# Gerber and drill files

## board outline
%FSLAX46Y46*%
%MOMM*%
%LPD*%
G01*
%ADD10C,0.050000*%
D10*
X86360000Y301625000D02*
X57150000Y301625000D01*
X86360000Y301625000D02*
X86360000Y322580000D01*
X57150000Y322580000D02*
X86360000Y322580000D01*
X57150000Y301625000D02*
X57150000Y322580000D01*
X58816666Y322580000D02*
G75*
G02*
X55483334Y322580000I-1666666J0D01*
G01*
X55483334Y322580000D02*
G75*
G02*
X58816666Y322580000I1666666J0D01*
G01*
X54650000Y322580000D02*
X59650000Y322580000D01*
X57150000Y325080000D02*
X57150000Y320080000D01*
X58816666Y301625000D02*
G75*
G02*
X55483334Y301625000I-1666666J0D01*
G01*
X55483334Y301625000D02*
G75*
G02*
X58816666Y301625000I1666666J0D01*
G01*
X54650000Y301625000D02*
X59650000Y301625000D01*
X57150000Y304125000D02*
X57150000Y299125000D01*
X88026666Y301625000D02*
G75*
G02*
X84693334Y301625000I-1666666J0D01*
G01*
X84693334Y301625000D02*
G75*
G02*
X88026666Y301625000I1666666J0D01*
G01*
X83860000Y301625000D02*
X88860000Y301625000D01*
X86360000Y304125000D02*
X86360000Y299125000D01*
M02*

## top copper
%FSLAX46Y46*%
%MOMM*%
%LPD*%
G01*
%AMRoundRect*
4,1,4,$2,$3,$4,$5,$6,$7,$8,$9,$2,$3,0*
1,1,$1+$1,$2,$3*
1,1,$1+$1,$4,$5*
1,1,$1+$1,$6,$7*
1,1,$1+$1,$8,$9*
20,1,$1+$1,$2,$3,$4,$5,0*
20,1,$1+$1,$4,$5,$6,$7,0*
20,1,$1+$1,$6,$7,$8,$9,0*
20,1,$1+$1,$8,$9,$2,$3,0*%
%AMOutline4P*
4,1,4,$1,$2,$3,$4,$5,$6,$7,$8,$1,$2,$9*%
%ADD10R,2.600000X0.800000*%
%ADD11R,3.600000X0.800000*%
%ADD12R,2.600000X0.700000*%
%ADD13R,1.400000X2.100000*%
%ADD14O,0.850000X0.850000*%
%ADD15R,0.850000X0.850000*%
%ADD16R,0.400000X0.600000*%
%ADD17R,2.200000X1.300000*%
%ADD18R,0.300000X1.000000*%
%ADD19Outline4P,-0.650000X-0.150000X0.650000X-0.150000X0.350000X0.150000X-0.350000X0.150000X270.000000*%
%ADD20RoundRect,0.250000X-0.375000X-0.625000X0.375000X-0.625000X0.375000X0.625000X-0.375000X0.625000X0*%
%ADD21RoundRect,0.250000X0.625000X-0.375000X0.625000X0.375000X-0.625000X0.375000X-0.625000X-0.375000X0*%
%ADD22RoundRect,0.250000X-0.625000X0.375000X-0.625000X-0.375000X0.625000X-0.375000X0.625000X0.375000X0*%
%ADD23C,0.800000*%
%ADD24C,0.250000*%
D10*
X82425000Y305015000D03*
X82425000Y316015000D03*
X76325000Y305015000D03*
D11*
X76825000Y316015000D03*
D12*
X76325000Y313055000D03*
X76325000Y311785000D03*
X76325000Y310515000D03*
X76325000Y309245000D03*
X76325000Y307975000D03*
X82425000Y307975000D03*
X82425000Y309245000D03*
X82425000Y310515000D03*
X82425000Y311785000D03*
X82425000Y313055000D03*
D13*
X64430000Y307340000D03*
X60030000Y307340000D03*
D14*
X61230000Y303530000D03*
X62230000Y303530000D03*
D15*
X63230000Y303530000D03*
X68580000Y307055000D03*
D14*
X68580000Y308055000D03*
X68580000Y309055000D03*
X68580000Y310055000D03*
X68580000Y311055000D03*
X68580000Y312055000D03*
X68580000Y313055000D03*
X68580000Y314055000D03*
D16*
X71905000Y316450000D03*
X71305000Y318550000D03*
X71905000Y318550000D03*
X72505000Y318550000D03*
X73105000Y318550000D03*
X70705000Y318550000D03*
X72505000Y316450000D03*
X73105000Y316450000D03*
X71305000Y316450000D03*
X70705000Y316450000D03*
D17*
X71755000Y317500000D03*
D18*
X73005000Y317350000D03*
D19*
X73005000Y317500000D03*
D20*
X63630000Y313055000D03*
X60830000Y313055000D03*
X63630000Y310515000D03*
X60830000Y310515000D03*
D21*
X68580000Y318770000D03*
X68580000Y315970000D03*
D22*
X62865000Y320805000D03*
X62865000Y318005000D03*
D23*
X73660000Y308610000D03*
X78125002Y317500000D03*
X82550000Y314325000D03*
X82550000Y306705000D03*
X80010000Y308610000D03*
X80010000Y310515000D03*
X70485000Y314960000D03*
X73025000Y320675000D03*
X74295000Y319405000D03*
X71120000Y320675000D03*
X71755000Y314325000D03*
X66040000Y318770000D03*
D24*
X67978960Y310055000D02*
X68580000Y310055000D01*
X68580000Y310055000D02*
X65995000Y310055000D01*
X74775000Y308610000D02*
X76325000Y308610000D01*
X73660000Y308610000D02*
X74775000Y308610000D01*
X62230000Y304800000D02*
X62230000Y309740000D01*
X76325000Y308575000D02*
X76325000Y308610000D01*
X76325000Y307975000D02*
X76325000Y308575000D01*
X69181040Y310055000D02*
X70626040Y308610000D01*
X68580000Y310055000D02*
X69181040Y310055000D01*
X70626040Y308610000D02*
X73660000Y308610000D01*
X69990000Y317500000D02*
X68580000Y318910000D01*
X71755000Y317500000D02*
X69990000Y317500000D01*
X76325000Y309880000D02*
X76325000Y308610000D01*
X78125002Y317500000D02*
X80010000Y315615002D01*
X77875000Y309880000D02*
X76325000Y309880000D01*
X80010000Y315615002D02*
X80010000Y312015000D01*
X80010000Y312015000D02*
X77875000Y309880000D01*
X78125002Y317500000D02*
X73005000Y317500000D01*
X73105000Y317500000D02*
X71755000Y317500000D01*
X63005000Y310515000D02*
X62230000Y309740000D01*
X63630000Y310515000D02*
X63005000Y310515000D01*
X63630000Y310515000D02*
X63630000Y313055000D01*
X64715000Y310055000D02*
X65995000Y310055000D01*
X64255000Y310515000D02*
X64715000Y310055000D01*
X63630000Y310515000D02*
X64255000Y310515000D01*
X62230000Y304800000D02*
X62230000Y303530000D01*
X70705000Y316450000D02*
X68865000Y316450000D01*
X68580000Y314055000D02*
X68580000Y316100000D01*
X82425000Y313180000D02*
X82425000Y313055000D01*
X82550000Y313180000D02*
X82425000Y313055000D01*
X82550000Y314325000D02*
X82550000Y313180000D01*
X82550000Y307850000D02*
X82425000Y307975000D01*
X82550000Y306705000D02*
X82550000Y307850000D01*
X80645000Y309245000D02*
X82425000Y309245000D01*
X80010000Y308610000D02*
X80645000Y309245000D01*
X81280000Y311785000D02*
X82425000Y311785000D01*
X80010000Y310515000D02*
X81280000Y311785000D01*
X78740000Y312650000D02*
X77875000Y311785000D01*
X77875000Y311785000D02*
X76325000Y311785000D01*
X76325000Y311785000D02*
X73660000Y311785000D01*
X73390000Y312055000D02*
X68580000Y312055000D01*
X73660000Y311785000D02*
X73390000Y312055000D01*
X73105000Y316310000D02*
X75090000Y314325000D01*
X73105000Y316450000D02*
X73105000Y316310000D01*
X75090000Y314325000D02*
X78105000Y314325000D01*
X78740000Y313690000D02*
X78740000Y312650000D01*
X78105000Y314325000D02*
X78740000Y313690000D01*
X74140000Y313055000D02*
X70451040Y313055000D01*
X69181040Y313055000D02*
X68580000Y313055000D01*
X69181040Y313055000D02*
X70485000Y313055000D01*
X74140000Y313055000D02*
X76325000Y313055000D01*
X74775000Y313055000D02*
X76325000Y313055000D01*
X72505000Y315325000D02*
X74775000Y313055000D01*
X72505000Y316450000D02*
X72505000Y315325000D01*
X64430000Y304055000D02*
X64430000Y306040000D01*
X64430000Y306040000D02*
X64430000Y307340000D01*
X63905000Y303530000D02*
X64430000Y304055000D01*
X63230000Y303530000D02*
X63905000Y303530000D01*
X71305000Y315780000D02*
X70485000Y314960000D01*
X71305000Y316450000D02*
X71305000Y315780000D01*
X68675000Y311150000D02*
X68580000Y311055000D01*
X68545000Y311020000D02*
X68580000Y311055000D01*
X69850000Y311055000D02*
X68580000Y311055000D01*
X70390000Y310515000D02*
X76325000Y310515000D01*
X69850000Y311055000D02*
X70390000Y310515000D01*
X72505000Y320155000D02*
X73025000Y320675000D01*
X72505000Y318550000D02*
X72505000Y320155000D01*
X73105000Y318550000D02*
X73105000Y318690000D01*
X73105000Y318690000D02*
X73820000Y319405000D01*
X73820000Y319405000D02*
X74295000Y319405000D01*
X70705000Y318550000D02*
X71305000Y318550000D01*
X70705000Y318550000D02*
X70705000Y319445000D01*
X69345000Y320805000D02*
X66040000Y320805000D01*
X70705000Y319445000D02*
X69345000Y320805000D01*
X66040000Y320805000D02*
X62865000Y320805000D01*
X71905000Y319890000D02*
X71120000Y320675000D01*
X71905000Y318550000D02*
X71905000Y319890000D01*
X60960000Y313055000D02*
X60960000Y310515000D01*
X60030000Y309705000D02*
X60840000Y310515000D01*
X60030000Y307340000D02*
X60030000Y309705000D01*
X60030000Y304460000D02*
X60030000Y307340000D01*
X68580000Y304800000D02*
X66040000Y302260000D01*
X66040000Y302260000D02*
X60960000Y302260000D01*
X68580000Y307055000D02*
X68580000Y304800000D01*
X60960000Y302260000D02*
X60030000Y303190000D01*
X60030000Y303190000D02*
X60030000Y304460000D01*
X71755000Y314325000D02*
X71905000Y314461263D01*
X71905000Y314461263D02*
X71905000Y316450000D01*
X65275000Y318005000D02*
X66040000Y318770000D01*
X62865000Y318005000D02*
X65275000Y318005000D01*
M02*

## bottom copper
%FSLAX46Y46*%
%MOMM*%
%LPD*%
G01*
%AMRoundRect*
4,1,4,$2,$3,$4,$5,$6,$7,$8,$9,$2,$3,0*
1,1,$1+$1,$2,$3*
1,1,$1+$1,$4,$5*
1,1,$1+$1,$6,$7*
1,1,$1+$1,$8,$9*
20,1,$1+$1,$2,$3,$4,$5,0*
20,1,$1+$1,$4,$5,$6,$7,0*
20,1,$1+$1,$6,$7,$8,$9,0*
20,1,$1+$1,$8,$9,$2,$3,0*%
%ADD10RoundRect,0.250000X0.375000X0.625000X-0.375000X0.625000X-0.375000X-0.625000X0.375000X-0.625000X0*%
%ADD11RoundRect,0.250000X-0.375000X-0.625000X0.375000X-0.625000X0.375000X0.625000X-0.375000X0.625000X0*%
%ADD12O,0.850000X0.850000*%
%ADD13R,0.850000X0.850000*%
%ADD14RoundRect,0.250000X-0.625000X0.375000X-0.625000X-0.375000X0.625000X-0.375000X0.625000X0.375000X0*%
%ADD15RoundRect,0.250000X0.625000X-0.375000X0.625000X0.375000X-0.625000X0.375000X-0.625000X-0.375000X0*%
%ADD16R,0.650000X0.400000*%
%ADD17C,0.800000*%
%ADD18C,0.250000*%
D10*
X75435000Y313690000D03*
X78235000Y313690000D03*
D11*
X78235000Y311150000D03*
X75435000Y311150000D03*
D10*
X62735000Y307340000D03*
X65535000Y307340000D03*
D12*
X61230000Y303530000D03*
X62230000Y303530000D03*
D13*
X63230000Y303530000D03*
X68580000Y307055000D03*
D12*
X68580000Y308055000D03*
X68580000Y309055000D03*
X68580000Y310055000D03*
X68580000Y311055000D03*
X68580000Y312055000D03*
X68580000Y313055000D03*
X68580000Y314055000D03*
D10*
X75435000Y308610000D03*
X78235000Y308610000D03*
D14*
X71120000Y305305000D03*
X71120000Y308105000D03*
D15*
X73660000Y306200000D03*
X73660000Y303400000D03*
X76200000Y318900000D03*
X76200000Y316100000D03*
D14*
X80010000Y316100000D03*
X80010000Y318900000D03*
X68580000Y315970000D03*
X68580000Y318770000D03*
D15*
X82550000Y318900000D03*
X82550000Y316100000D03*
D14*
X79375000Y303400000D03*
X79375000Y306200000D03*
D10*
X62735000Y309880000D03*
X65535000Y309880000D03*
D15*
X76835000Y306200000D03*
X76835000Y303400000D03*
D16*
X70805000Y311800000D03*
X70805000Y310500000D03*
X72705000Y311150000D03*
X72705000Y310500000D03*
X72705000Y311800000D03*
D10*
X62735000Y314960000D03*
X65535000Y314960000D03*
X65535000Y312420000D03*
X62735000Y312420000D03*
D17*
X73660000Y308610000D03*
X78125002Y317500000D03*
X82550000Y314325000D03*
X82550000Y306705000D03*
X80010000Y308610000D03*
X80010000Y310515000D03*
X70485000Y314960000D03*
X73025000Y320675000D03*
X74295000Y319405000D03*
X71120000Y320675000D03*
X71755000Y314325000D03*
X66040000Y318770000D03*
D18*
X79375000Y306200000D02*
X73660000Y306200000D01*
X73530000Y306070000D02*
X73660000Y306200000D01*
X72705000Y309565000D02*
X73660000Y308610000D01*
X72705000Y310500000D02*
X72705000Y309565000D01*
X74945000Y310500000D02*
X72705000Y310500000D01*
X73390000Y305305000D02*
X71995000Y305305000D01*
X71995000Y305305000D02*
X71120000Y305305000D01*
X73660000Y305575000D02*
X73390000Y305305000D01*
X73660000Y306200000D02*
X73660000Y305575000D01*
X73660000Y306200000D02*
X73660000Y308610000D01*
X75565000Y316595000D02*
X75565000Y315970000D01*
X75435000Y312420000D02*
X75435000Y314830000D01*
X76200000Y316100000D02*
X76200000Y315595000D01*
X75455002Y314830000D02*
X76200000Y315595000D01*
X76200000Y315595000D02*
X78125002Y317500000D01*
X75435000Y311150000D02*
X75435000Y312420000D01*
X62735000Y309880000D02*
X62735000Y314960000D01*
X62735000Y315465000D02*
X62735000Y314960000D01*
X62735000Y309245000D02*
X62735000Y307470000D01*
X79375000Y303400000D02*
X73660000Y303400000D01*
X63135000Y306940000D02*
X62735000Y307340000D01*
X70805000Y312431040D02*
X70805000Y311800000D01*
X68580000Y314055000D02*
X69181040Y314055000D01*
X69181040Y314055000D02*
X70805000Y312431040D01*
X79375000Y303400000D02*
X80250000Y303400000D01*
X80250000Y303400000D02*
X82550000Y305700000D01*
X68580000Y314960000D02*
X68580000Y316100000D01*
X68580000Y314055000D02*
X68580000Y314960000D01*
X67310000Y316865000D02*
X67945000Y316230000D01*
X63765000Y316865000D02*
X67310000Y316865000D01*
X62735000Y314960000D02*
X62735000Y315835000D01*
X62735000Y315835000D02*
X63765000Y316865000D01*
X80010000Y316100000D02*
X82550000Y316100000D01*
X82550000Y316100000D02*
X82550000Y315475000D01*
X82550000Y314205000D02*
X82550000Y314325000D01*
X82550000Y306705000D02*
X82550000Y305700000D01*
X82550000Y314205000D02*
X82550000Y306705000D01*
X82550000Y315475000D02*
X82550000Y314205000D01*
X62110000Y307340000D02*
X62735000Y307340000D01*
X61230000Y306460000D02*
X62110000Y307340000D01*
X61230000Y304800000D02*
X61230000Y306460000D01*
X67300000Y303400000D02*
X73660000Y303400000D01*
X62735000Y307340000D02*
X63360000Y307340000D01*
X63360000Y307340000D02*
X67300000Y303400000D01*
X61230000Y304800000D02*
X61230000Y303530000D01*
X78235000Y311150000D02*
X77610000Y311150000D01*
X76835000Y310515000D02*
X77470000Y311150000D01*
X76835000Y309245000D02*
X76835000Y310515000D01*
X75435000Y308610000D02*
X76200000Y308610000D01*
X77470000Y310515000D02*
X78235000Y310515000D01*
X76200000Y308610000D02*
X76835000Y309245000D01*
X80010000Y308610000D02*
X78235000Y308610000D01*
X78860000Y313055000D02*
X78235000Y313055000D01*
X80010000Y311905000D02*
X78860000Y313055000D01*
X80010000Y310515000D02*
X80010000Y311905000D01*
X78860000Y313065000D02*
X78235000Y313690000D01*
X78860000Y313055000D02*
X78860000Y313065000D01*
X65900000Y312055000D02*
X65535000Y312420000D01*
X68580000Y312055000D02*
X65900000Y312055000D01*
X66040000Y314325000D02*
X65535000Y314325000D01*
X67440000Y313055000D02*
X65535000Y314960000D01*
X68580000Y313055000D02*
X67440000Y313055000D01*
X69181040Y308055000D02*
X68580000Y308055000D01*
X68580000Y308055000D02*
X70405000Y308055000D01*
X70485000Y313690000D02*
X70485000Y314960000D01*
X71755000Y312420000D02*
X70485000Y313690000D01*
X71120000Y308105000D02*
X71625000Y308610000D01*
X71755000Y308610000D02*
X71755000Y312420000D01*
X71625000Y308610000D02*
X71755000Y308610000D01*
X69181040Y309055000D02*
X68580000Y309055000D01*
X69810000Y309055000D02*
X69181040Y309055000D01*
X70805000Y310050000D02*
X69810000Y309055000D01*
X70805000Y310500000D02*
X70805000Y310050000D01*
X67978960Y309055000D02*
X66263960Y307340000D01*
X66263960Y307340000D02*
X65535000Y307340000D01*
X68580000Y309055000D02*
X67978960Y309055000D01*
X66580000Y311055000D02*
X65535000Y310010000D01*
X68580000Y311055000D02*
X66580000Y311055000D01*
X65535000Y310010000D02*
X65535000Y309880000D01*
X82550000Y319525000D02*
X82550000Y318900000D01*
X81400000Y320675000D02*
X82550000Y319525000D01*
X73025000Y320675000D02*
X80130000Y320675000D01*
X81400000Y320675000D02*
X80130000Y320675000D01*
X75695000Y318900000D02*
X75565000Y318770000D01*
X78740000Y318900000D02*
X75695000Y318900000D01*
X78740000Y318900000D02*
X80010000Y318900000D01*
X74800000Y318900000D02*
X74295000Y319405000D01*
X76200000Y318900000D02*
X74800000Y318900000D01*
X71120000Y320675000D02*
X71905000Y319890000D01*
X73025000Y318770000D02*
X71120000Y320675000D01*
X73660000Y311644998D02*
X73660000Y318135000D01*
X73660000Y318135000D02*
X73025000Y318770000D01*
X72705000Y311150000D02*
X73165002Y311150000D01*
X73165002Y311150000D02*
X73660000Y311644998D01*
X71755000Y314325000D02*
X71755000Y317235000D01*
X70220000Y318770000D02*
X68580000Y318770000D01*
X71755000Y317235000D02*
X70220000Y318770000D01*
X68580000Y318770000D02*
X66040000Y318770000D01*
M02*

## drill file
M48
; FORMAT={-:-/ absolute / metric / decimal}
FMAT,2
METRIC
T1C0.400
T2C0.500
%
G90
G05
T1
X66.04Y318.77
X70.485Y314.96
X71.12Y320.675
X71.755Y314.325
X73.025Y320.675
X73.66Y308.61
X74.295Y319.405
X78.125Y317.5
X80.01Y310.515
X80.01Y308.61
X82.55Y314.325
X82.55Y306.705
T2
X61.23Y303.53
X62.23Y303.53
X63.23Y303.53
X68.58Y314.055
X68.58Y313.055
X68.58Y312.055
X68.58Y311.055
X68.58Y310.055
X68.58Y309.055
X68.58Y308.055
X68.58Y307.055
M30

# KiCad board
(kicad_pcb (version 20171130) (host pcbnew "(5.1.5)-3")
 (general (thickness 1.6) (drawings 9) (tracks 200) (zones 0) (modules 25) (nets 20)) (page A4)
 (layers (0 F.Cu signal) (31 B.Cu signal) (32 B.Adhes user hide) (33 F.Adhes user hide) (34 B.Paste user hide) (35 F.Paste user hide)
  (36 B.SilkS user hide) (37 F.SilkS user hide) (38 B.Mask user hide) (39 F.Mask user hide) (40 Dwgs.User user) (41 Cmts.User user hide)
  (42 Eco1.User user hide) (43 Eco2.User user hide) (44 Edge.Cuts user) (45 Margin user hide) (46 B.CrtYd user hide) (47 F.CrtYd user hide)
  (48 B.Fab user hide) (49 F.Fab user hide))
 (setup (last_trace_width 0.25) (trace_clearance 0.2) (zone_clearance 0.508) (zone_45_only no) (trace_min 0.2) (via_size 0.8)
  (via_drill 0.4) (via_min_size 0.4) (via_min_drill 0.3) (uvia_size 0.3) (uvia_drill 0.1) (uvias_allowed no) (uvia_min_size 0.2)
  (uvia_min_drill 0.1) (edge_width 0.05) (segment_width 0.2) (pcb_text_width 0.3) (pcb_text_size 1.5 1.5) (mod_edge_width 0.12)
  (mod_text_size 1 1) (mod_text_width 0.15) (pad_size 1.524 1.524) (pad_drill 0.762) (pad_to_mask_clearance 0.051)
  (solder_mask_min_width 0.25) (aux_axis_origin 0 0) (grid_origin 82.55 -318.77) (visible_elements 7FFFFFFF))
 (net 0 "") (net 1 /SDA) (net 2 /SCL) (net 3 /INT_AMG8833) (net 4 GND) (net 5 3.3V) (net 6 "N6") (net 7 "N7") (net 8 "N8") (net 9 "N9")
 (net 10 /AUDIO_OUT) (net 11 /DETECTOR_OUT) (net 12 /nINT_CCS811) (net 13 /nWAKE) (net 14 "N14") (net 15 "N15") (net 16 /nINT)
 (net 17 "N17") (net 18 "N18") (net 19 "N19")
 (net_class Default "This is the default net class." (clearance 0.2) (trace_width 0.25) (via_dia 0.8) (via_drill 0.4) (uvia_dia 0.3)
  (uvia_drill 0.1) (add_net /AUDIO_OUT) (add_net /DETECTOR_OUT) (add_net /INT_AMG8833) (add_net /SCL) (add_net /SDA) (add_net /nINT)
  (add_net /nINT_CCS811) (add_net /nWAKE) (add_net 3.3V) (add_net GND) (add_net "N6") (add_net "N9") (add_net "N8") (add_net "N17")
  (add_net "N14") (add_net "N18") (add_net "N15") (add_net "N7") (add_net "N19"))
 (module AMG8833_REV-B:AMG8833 (layer F.Cu) (at 79.375 -310.515 270)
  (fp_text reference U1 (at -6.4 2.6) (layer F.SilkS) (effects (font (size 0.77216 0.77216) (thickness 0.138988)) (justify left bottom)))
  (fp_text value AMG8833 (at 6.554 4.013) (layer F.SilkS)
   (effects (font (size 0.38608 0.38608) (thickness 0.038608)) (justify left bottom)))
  (pad 8 smd rect (at 5.5 -3.05) (size 2.6 0.8) (layers F.Cu F.Paste F.Mask) (solder_mask_margin 0.0508))
  (pad 14 smd rect (at -5.5 -3.05) (size 2.6 0.8) (layers F.Cu F.Paste F.Mask) (solder_mask_margin 0.0508))
  (pad 7 smd rect (at 5.5 3.05) (size 2.6 0.8) (layers F.Cu F.Paste F.Mask) (solder_mask_margin 0.0508))
  (pad 1 smd rect (at -5.5 2.55) (size 3.6 0.8) (layers F.Cu F.Paste F.Mask) (solder_mask_margin 0.0508))
  (pad 2 smd rect (at -2.54 3.05) (size 2.6 0.7) (layers F.Cu F.Paste F.Mask) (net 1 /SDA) (solder_mask_margin 0.0508))
  (pad 3 smd rect (at -1.27 3.05) (size 2.6 0.7) (layers F.Cu F.Paste F.Mask) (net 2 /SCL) (solder_mask_margin 0.0508))
  (pad 4 smd rect (at 0 3.05) (size 2.6 0.7) (layers F.Cu F.Paste F.Mask) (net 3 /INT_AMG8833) (solder_mask_margin 0.0508))
  (pad 5 smd rect (at 1.27 3.05) (size 2.6 0.7) (layers F.Cu F.Paste F.Mask) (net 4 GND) (solder_mask_margin 0.0508))
  (pad 6 smd rect (at 2.54 3.05) (size 2.6 0.7) (layers F.Cu F.Paste F.Mask) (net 4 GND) (solder_mask_margin 0.0508))
  (pad 9 smd rect (at 2.54 -3.05) (size 2.6 0.7) (layers F.Cu F.Paste F.Mask) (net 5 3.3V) (solder_mask_margin 0.0508))
  (pad 10 smd rect (at 1.27 -3.05) (size 2.6 0.7) (layers F.Cu F.Paste F.Mask) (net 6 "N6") (solder_mask_margin 0.0508))
  (pad 11 smd rect (at 0 -3.05) (size 2.6 0.7) (layers F.Cu F.Paste F.Mask) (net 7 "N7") (solder_mask_margin 0.0508))
  (pad 12 smd rect (at -1.27 -3.05) (size 2.6 0.7) (layers F.Cu F.Paste F.Mask) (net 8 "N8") (solder_mask_margin 0.0508))
  (pad 13 smd rect (at -2.54 -3.05) (size 2.6 0.7) (layers F.Cu F.Paste F.Mask) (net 5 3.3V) (solder_mask_margin 0.0508)))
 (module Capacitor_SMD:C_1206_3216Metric (layer B.Cu) (at 76.835 -313.69 180)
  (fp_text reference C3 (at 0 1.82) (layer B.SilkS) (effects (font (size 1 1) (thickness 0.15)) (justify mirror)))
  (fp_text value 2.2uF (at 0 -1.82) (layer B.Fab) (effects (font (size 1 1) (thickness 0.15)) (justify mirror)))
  (pad 2 smd roundrect (at 1.4 0 180) (size 1.25 1.75) (layers B.Cu B.Paste B.Mask) (roundrect_rratio 0.2) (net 4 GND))
  (pad 1 smd roundrect (at -1.4 0 180) (size 1.25 1.75) (layers B.Cu B.Paste B.Mask) (roundrect_rratio 0.2) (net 8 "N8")))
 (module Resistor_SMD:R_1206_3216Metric (layer B.Cu) (at 76.835 -311.15)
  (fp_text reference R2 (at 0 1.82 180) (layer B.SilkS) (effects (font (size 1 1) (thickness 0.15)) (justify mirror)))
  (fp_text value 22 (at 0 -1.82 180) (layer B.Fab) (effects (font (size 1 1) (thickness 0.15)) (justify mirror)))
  (pad 2 smd roundrect (at 1.4 0) (size 1.25 1.75) (layers B.Cu B.Paste B.Mask) (roundrect_rratio 0.2) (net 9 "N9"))
  (pad 1 smd roundrect (at -1.4 0) (size 1.25 1.75) (layers B.Cu B.Paste B.Mask) (roundrect_rratio 0.2) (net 4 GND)))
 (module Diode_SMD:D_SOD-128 (layer F.Cu) (at 62.23 -307.34)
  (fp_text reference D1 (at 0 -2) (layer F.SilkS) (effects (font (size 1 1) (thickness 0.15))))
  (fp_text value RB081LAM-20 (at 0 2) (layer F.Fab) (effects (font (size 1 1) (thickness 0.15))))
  (pad 2 smd rect (at 2.2 0) (size 1.4 2.1) (layers F.Cu F.Paste F.Mask) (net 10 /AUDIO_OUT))
  (pad 1 smd rect (at -2.2 0) (size 1.4 2.1) (layers F.Cu F.Paste F.Mask) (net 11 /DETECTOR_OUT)))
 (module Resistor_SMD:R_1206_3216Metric (layer B.Cu) (at 64.135 -307.34 180)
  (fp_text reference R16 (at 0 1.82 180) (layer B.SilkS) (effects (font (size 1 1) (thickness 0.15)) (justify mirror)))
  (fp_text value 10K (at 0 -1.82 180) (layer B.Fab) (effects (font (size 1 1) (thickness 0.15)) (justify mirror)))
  (pad 2 smd roundrect (at 1.4 0 180) (size 1.25 1.75) (layers B.Cu B.Paste B.Mask) (roundrect_rratio 0.2) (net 5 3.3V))
  (pad 1 smd roundrect (at -1.4 0 180) (size 1.25 1.75) (layers B.Cu B.Paste B.Mask) (roundrect_rratio 0.2) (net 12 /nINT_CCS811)))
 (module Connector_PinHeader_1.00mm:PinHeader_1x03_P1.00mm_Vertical (layer F.Cu) (at 63.23 -303.53 270)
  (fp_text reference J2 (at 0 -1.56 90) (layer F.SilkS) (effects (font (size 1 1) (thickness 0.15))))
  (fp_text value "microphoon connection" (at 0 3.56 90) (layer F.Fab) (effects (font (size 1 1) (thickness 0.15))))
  (pad 3 thru_hole oval (at 0 2 270) (size 0.85 0.85) (drill 0.5) (layers *.Cu *.Mask) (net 5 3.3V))
  (pad 2 thru_hole oval (at 0 1 270) (size 0.85 0.85) (drill 0.5) (layers *.Cu *.Mask) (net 4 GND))
  (pad 1 thru_hole rect (at 0 0 270) (size 0.85 0.85) (drill 0.5) (layers *.Cu *.Mask) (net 10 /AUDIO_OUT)))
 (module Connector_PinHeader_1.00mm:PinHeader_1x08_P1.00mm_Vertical (layer F.Cu) (at 68.58 -307.055 180)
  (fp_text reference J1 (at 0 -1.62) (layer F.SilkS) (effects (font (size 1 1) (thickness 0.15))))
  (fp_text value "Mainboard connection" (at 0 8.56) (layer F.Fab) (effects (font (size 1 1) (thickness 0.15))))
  (pad 1 thru_hole rect (at 0 0 180) (size 0.85 0.85) (drill 0.5) (layers *.Cu *.Mask) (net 11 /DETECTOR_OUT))
  (pad 2 thru_hole oval (at 0 1 180) (size 0.85 0.85) (drill 0.5) (layers *.Cu *.Mask) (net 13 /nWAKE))
  (pad 3 thru_hole oval (at 0 2 180) (size 0.85 0.85) (drill 0.5) (layers *.Cu *.Mask) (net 12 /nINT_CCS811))
  (pad 4 thru_hole oval (at 0 3 180) (size 0.85 0.85) (drill 0.5) (layers *.Cu *.Mask) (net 4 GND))
  (pad 5 thru_hole oval (at 0 4 180) (size 0.85 0.85) (drill 0.5) (layers *.Cu *.Mask) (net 3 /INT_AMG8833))
  (pad 6 thru_hole oval (at 0 5 180) (size 0.85 0.85) (drill 0.5) (layers *.Cu *.Mask) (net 2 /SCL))
  (pad 7 thru_hole oval (at 0 6 180) (size 0.85 0.85) (drill 0.5) (layers *.Cu *.Mask) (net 1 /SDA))
  (pad 8 thru_hole oval (at 0 7 180) (size 0.85 0.85) (drill 0.5) (layers *.Cu *.Mask) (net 5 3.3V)))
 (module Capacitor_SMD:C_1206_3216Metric (layer B.Cu) (at 76.835 -308.61 180)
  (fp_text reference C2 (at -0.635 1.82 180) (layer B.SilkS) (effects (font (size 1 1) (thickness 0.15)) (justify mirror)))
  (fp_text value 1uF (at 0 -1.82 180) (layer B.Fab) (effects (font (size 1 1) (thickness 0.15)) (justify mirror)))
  (pad 2 smd roundrect (at 1.4 0 180) (size 1.25 1.75) (layers B.Cu B.Paste B.Mask) (roundrect_rratio 0.2) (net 9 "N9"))
  (pad 1 smd roundrect (at -1.4 0 180) (size 1.25 1.75) (layers B.Cu B.Paste B.Mask) (roundrect_rratio 0.2) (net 6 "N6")))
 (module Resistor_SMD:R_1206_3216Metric (layer B.Cu) (at 71.12 -306.705 270)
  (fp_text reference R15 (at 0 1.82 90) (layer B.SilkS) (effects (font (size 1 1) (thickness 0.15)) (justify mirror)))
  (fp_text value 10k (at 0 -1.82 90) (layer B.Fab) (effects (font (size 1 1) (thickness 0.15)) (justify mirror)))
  (pad 2 smd roundrect (at 1.4 0 270) (size 1.25 1.75) (layers B.Cu B.Paste B.Mask) (roundrect_rratio 0.2) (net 4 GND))
  (pad 1 smd roundrect (at -1.4 0 270) (size 1.25 1.75) (layers B.Cu B.Paste B.Mask) (roundrect_rratio 0.2) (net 13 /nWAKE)))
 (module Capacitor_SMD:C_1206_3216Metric (layer B.Cu) (at 73.66 -304.8 90)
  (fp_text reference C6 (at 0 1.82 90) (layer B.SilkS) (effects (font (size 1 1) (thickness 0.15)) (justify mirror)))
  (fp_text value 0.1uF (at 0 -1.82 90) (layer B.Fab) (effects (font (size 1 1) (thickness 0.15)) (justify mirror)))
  (pad 2 smd roundrect (at 1.4 0 90) (size 1.25 1.75) (layers B.Cu B.Paste B.Mask) (roundrect_rratio 0.2) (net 4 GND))
  (pad 1 smd roundrect (at -1.4 0 90) (size 1.25 1.75) (layers B.Cu B.Paste B.Mask) (roundrect_rratio 0.2) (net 5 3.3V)))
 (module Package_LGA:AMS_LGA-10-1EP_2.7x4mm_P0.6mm (layer F.Cu) (at 71.905 -317.5 270)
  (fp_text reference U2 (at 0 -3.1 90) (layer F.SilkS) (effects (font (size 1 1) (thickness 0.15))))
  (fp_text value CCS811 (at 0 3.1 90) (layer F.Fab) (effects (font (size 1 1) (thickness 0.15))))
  (pad 8 smd rect (at 1.05 0 270) (size 0.6 0.4) (layers F.Cu F.Paste F.Mask) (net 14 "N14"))
  (pad 4 smd rect (at -1.05 0.6 270) (size 0.6 0.4) (layers F.Cu F.Paste F.Mask) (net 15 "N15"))
  (pad 3 smd rect (at -1.05 0 270) (size 0.6 0.4) (layers F.Cu F.Paste F.Mask) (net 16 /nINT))
  (pad 2 smd rect (at -1.05 -0.6 270) (size 0.6 0.4) (layers F.Cu F.Paste F.Mask) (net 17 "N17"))
  (pad 1 smd rect (at -1.05 -1.2 270) (size 0.6 0.4) (layers F.Cu F.Paste F.Mask) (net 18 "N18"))
  (pad 5 smd rect (at -1.05 1.2 270) (size 0.6 0.4) (layers F.Cu F.Paste F.Mask) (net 15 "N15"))
  (pad 9 smd rect (at 1.05 -0.6 270) (size 0.6 0.4) (layers F.Cu F.Paste F.Mask) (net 1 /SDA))
  (pad 10 smd rect (at 1.05 -1.2 270) (size 0.6 0.4) (layers F.Cu F.Paste F.Mask) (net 2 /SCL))
  (pad 7 smd rect (at 1.05 0.6 270) (size 0.6 0.4) (layers F.Cu F.Paste F.Mask) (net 13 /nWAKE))
  (pad 6 smd rect (at 1.05 1.2 270) (size 0.6 0.4) (layers F.Cu F.Paste F.Mask) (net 5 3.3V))
  (pad 11 smd rect (at 0 0.15 270) (size 1.3 2.2) (layers F.Cu F.Paste F.Mask) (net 4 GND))
  (pad 11 smd rect (at 0.15 -1.1 270) (size 1 0.3) (layers F.Cu F.Paste F.Mask) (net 4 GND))
  (pad 11 smd trapezoid (at 0 -1.1 270) (size 1 0.3) (rect_delta 0 0.3) (layers F.Cu F.Paste F.Mask) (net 4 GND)))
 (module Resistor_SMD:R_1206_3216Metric (layer F.Cu) (at 62.23 -313.055)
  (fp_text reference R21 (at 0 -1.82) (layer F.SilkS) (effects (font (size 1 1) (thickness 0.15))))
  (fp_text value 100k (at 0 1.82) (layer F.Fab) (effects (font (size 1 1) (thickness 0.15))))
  (pad 2 smd roundrect (at 1.4 0) (size 1.25 1.75) (layers F.Cu F.Paste F.Mask) (roundrect_rratio 0.2) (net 4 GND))
  (pad 1 smd roundrect (at -1.4 0) (size 1.25 1.75) (layers F.Cu F.Paste F.Mask) (roundrect_rratio 0.2) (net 11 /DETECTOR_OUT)))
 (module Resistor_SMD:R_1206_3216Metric (layer B.Cu) (at 76.2 -317.5 90)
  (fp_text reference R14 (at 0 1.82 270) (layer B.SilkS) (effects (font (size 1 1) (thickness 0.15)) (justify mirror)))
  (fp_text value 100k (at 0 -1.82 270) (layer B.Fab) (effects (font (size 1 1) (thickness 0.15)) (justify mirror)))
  (pad 2 smd roundrect (at 1.4 0 90) (size 1.25 1.75) (layers B.Cu B.Paste B.Mask) (roundrect_rratio 0.2) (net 18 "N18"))
  (pad 1 smd roundrect (at -1.4 0 90) (size 1.25 1.75) (layers B.Cu B.Paste B.Mask) (roundrect_rratio 0.2) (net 4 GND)))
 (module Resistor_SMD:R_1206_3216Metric (layer B.Cu) (at 80.01 -317.5 270)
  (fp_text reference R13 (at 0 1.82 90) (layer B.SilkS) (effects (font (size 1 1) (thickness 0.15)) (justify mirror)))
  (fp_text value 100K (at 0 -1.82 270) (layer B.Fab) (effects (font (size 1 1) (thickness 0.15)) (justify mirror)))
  (pad 2 smd roundrect (at 1.4 0 270) (size 1.25 1.75) (layers B.Cu B.Paste B.Mask) (roundrect_rratio 0.2) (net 5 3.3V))
  (pad 1 smd roundrect (at -1.4 0 270) (size 1.25 1.75) (layers B.Cu B.Paste B.Mask) (roundrect_rratio 0.2) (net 18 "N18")))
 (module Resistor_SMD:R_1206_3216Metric (layer B.Cu) (at 68.58 -317.37 270)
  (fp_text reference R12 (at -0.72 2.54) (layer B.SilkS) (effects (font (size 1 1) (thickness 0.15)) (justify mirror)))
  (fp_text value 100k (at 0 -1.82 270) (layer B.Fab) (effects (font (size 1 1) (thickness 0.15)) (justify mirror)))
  (pad 2 smd roundrect (at 1.4 0 270) (size 1.25 1.75) (layers B.Cu B.Paste B.Mask) (roundrect_rratio 0.2) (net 5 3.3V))
  (pad 1 smd roundrect (at -1.4 0 270) (size 1.25 1.75) (layers B.Cu B.Paste B.Mask) (roundrect_rratio 0.2) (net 14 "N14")))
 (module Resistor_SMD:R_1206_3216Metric (layer B.Cu) (at 82.55 -317.5 90)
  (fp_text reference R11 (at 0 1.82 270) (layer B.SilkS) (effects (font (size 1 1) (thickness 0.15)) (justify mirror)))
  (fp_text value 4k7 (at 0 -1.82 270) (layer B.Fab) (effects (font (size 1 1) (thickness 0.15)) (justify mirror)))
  (pad 2 smd roundrect (at 1.4 0 90) (size 1.25 1.75) (layers B.Cu B.Paste B.Mask) (roundrect_rratio 0.2) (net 17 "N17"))
  (pad 1 smd roundrect (at -1.4 0 90) (size 1.25 1.75) (layers B.Cu B.Paste B.Mask) (roundrect_rratio 0.2) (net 5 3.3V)))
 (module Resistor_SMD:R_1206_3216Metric (layer B.Cu) (at 79.375 -304.8 270)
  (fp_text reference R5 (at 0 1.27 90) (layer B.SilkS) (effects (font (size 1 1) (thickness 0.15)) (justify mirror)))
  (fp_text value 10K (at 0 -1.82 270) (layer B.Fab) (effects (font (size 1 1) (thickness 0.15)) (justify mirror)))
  (pad 2 smd roundrect (at 1.4 0 270) (size 1.25 1.75) (layers B.Cu B.Paste B.Mask) (roundrect_rratio 0.2) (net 5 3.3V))
  (pad 1 smd roundrect (at -1.4 0 270) (size 1.25 1.75) (layers B.Cu B.Paste B.Mask) (roundrect_rratio 0.2) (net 4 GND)))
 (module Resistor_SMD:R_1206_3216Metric (layer B.Cu) (at 64.135 -309.88 180)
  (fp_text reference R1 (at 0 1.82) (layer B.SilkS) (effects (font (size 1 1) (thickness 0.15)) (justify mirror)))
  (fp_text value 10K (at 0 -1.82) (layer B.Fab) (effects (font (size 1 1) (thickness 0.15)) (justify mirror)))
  (pad 2 smd roundrect (at 1.4 0 180) (size 1.25 1.75) (layers B.Cu B.Paste B.Mask) (roundrect_rratio 0.2) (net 5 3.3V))
  (pad 1 smd roundrect (at -1.4 0 180) (size 1.25 1.75) (layers B.Cu B.Paste B.Mask) (roundrect_rratio 0.2) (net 3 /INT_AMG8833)))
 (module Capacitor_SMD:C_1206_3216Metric (layer F.Cu) (at 62.23 -310.515)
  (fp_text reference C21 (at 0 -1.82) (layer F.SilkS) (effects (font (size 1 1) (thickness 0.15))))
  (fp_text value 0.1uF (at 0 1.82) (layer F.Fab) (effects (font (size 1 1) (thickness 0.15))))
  (pad 2 smd roundrect (at 1.4 0) (size 1.25 1.75) (layers F.Cu F.Paste F.Mask) (roundrect_rratio 0.2) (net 4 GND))
  (pad 1 smd roundrect (at -1.4 0) (size 1.25 1.75) (layers F.Cu F.Paste F.Mask) (roundrect_rratio 0.2) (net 11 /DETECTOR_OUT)))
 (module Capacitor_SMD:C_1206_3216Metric (layer F.Cu) (at 68.58 -317.37 90)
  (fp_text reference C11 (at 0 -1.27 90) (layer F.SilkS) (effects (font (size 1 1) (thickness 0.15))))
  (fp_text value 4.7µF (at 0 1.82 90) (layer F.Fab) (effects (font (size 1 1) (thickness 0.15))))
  (pad 2 smd roundrect (at 1.4 0 90) (size 1.25 1.75) (layers F.Cu F.Paste F.Mask) (roundrect_rratio 0.2) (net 4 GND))
  (pad 1 smd roundrect (at -1.4 0 90) (size 1.25 1.75) (layers F.Cu F.Paste F.Mask) (roundrect_rratio 0.2) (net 5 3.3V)))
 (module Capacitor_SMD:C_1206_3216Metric (layer B.Cu) (at 76.835 -304.8 90)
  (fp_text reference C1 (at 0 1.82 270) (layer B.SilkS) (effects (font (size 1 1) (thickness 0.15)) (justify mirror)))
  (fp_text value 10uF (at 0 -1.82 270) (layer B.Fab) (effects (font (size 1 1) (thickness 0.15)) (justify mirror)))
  (pad 2 smd roundrect (at 1.4 0 90) (size 1.25 1.75) (layers B.Cu B.Paste B.Mask) (roundrect_rratio 0.2) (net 4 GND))
  (pad 1 smd roundrect (at -1.4 0 90) (size 1.25 1.75) (layers B.Cu B.Paste B.Mask) (roundrect_rratio 0.2) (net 5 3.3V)))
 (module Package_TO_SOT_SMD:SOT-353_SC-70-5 (layer B.Cu) (at 71.755 -311.15 180)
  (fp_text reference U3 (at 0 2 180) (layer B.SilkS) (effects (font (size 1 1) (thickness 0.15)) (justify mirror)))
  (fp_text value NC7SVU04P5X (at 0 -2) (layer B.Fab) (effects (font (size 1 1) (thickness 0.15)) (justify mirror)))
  (pad 5 smd rect (at 0.95 0.65 180) (size 0.65 0.4) (layers B.Cu B.Paste B.Mask) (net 5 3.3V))
  (pad 4 smd rect (at 0.95 -0.65 180) (size 0.65 0.4) (layers B.Cu B.Paste B.Mask) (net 12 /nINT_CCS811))
  (pad 2 smd rect (at -0.95 0 180) (size 0.65 0.4) (layers B.Cu B.Paste B.Mask) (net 16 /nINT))
  (pad 3 smd rect (at -0.95 -0.65 180) (size 0.65 0.4) (layers B.Cu B.Paste B.Mask) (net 4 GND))
  (pad 1 smd rect (at -0.95 0.65 180) (size 0.65 0.4) (layers B.Cu B.Paste B.Mask) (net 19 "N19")))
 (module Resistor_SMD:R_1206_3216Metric (layer B.Cu) (at 64.135 -314.96 180)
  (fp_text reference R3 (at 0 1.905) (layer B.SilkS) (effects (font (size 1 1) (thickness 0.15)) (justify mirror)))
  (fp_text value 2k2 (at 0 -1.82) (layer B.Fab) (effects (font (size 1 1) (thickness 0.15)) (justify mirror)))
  (pad 2 smd roundrect (at 1.4 0 180) (size 1.25 1.75) (layers B.Cu B.Paste B.Mask) (roundrect_rratio 0.2) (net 5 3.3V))
  (pad 1 smd roundrect (at -1.4 0 180) (size 1.25 1.75) (layers B.Cu B.Paste B.Mask) (roundrect_rratio 0.2) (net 1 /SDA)))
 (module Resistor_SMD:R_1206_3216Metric (layer B.Cu) (at 64.135 -312.42 180)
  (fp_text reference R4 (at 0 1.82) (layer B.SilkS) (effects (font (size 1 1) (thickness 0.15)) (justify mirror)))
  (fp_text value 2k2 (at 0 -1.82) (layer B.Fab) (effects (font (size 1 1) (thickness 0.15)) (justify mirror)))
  (pad 1 smd roundrect (at -1.4 0 180) (size 1.25 1.75) (layers B.Cu B.Paste B.Mask) (roundrect_rratio 0.2) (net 2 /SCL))
  (pad 2 smd roundrect (at 1.4 0 180) (size 1.25 1.75) (layers B.Cu B.Paste B.Mask) (roundrect_rratio 0.2) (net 5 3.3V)))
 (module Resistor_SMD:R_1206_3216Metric (layer F.Cu) (at 62.865 -319.405 270)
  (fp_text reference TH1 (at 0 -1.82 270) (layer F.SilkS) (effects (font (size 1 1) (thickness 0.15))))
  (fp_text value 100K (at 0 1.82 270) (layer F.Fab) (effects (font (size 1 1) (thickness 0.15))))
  (pad 1 smd roundrect (at -1.4 0 270) (size 1.25 1.75) (layers F.Cu F.Paste F.Mask) (roundrect_rratio 0.2) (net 15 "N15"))
  (pad 2 smd roundrect (at 1.4 0 270) (size 1.25 1.75) (layers F.Cu F.Paste F.Mask) (roundrect_rratio 0.2) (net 14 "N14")))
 (gr_line (start 86.36 -301.625) (end 57.15 -301.625) (layer Edge.Cuts) (width 0.05))
 (gr_line (start 86.36 -301.625) (end 86.36 -322.58) (layer Edge.Cuts) (width 0.05))
 (gr_line (start 57.15 -322.58) (end 86.36 -322.58) (layer Edge.Cuts) (width 0.05))
 (gr_line (start 57.15 -301.625) (end 57.15 -322.58) (layer Edge.Cuts) (width 0.05))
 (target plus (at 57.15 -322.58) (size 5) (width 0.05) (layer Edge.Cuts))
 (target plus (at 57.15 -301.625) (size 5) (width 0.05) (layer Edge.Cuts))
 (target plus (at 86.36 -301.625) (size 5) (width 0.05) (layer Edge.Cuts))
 (segment (start 67.97896 -310.055) (end 68.58 -310.055) (width 0.25) (layer F.Cu) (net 4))
 (segment (start 79.375 -306.2) (end 73.66 -306.2) (width 0.25) (layer B.Cu) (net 4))
 (segment (start 68.58 -310.055) (end 65.995 -310.055) (width 0.25) (layer F.Cu) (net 4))
 (segment (start 74.775 -308.61) (end 76.325 -308.61) (width 0.25) (layer F.Cu) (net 4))
 (segment (start 73.66 -308.61) (end 74.775 -308.61) (width 0.25) (layer F.Cu) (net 4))
 (via (at 73.66 -308.61) (size 0.8) (drill 0.4) (layers F.Cu B.Cu) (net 4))
 (segment (start 73.53 -306.07) (end 73.66 -306.2) (width 0.25) (layer B.Cu) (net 4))
 (segment (start 62.23 -304.8) (end 62.23 -309.74) (width 0.25) (layer F.Cu) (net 4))
 (segment (start 76.325 -308.575) (end 76.325 -308.61) (width 0.25) (layer F.Cu) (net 4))
 (segment (start 76.325 -307.975) (end 76.325 -308.575) (width 0.25) (layer F.Cu) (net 4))
 (segment (start 69.18104 -310.055) (end 70.62604 -308.61) (width 0.25) (layer F.Cu) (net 4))
 (segment (start 68.58 -310.055) (end 69.18104 -310.055) (width 0.25) (layer F.Cu) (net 4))
 (segment (start 70.62604 -308.61) (end 73.66 -308.61) (width 0.25) (layer F.Cu) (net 4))
 (segment (start 69.99 -317.5) (end 68.58 -318.91) (width 0.25) (layer F.Cu) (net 4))
 (segment (start 71.755 -317.5) (end 69.99 -317.5) (width 0.25) (layer F.Cu) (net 4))
 (segment (start 72.705 -309.565) (end 73.66 -308.61) (width 0.25) (layer B.Cu) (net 4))
 (segment (start 72.705 -310.5) (end 72.705 -309.565) (width 0.25) (layer B.Cu) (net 4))
 (segment (start 74.945 -310.5) (end 72.705 -310.5) (width 0.25) (layer B.Cu) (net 4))
 (segment (start 73.39 -305.305) (end 71.995 -305.305) (width 0.25) (layer B.Cu) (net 4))
 (segment (start 71.995 -305.305) (end 71.12 -305.305) (width 0.25) (layer B.Cu) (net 4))
 (segment (start 73.66 -305.575) (end 73.39 -305.305) (width 0.25) (layer B.Cu) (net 4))
 (segment (start 73.66 -306.2) (end 73.66 -305.575) (width 0.25) (layer B.Cu) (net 4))
 (segment (start 73.66 -306.2) (end 73.66 -308.61) (width 0.25) (layer B.Cu) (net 4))
 (segment (start 76.325 -309.88) (end 76.325 -308.61) (width 0.25) (layer F.Cu) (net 4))
 (segment (start 78.125002 -317.5) (end 80.01 -315.615002) (width 0.25) (layer F.Cu) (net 4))
 (segment (start 77.875 -309.88) (end 76.325 -309.88) (width 0.25) (layer F.Cu) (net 4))
 (segment (start 80.01 -315.615002) (end 80.01 -312.015) (width 0.25) (layer F.Cu) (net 4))
 (segment (start 80.01 -312.015) (end 77.875 -309.88) (width 0.25) (layer F.Cu) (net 4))
 (segment (start 78.125002 -317.5) (end 73.005 -317.5) (width 0.25) (layer F.Cu) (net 4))
 (via (at 78.125002 -317.5) (size 0.8) (drill 0.4) (layers F.Cu B.Cu) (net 4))
 (segment (start 75.565 -316.595) (end 75.565 -315.97) (width 0.25) (layer B.Cu) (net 4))
 (segment (start 73.105 -317.5) (end 71.755 -317.5) (width 0.25) (layer F.Cu) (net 4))
 (segment (start 75.435 -312.42) (end 75.435 -314.83) (width 0.25) (layer B.Cu) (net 4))
 (segment (start 76.2 -316.1) (end 76.2 -315.595) (width 0.25) (layer B.Cu) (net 4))
 (segment (start 75.455002 -314.83) (end 76.2 -315.595) (width 0.25) (layer B.Cu) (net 4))
 (segment (start 76.2 -315.595) (end 78.125002 -317.5) (width 0.25) (layer B.Cu) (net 4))
 (segment (start 75.435 -311.15) (end 75.435 -312.42) (width 0.25) (layer B.Cu) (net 4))
 (segment (start 63.005 -310.515) (end 62.23 -309.74) (width 0.25) (layer F.Cu) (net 4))
 (segment (start 63.63 -310.515) (end 63.005 -310.515) (width 0.25) (layer F.Cu) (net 4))
 (segment (start 63.63 -310.515) (end 63.63 -313.055) (width 0.25) (layer F.Cu) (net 4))
 (segment (start 64.715 -310.055) (end 65.995 -310.055) (width 0.25) (layer F.Cu) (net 4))
 (segment (start 64.255 -310.515) (end 64.715 -310.055) (width 0.25) (layer F.Cu) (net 4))
 (segment (start 63.63 -310.515) (end 64.255 -310.515) (width 0.25) (layer F.Cu) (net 4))
 (segment (start 62.23 -304.8) (end 62.23 -303.53) (width 0.25) (layer F.Cu) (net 4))
 (segment (start 62.735 -309.88) (end 62.735 -314.96) (width 0.25) (layer B.Cu) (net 5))
 (segment (start 62.735 -315.465) (end 62.735 -314.96) (width 0.25) (layer B.Cu) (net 5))
 (segment (start 62.735 -309.245) (end 62.735 -307.47) (width 0.25) (layer B.Cu) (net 5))
 (segment (start 79.375 -303.4) (end 73.66 -303.4) (width 0.25) (layer B.Cu) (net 5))
 (segment (start 63.135 -306.94) (end 62.735 -307.34) (width 0.25) (layer B.Cu) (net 5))
 (segment (start 70.705 -316.45) (end 68.865 -316.45) (width 0.25) (layer F.Cu) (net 5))
 (segment (start 68.58 -314.055) (end 68.58 -316.1) (width 0.25) (layer F.Cu) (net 5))
 (segment (start 70.805 -312.43104) (end 70.805 -311.8) (width 0.25) (layer B.Cu) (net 5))
 (segment (start 68.58 -314.055) (end 69.18104 -314.055) (width 0.25) (layer B.Cu) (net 5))
 (segment (start 69.18104 -314.055) (end 70.805 -312.43104) (width 0.25) (layer B.Cu) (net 5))
 (segment (start 79.375 -303.4) (end 80.25 -303.4) (width 0.25) (layer B.Cu) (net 5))
 (segment (start 80.25 -303.4) (end 82.55 -305.7) (width 0.25) (layer B.Cu) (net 5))
 (segment (start 68.58 -314.96) (end 68.58 -316.1) (width 0.25) (layer B.Cu) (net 5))
 (segment (start 68.58 -314.055) (end 68.58 -314.96) (width 0.25) (layer B.Cu) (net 5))
 (segment (start 67.31 -316.865) (end 67.945 -316.23) (width 0.25) (layer B.Cu) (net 5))
 (segment (start 63.765 -316.865) (end 67.31 -316.865) (width 0.25) (layer B.Cu) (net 5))
 (segment (start 62.735 -314.96) (end 62.735 -315.835) (width 0.25) (layer B.Cu) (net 5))
 (segment (start 62.735 -315.835) (end 63.765 -316.865) (width 0.25) (layer B.Cu) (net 5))
 (segment (start 82.425 -313.18) (end 82.425 -313.055) (width 0.25) (layer F.Cu) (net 5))
 (segment (start 80.01 -316.1) (end 82.55 -316.1) (width 0.25) (layer B.Cu) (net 5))
 (segment (start 82.55 -316.1) (end 82.55 -315.475) (width 0.25) (layer B.Cu) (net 5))
 (via (at 82.55 -314.325) (size 0.8) (drill 0.4) (layers F.Cu B.Cu) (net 5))
 (segment (start 82.55 -314.205) (end 82.55 -314.325) (width 0.25) (layer B.Cu) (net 5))
 (segment (start 82.55 -313.18) (end 82.425 -313.055) (width 0.25) (layer F.Cu) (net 5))
 (segment (start 82.55 -314.325) (end 82.55 -313.18) (width 0.25) (layer F.Cu) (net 5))
 (via (at 82.55 -306.705) (size 0.8) (drill 0.4) (layers F.Cu B.Cu) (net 5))
 (segment (start 82.55 -306.705) (end 82.55 -305.7) (width 0.25) (layer B.Cu) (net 5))
 (segment (start 82.55 -314.205) (end 82.55 -306.705) (width 0.25) (layer B.Cu) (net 5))
 (segment (start 82.55 -307.85) (end 82.425 -307.975) (width 0.25) (layer F.Cu) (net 5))
 (segment (start 82.55 -306.705) (end 82.55 -307.85) (width 0.25) (layer F.Cu) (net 5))
 (segment (start 82.55 -315.475) (end 82.55 -314.205) (width 0.25) (layer B.Cu) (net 5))
 (segment (start 62.11 -307.34) (end 62.735 -307.34) (width 0.25) (layer B.Cu) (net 5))
 (segment (start 61.23 -306.46) (end 62.11 -307.34) (width 0.25) (layer B.Cu) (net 5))
 (segment (start 61.23 -304.8) (end 61.23 -306.46) (width 0.25) (layer B.Cu) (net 5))
 (segment (start 67.3 -303.4) (end 73.66 -303.4) (width 0.25) (layer B.Cu) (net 5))
 (segment (start 62.735 -307.34) (end 63.36 -307.34) (width 0.25) (layer B.Cu) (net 5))
 (segment (start 63.36 -307.34) (end 67.3 -303.4) (width 0.25) (layer B.Cu) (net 5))
 (segment (start 61.23 -304.8) (end 61.23 -303.53) (width 0.25) (layer B.Cu) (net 5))
 (segment (start 78.235 -311.15) (end 77.61 -311.15) (width 0.25) (layer B.Cu) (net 9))
 (segment (start 76.835 -310.515) (end 77.47 -311.15) (width 0.25) (layer B.Cu) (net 9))
 (segment (start 76.835 -309.245) (end 76.835 -310.515) (width 0.25) (layer B.Cu) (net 9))
 (segment (start 75.435 -308.61) (end 76.2 -308.61) (width 0.25) (layer B.Cu) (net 9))
 (segment (start 77.47 -310.515) (end 78.235 -310.515) (width 0.25) (layer B.Cu) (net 9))
 (segment (start 76.2 -308.61) (end 76.835 -309.245) (width 0.25) (layer B.Cu) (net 9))
 (segment (start 80.645 -309.245) (end 82.425 -309.245) (width 0.25) (layer F.Cu) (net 6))
 (via (at 80.01 -308.61) (size 0.8) (drill 0.4) (layers F.Cu B.Cu) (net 6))
 (segment (start 80.01 -308.61) (end 80.645 -309.245) (width 0.25) (layer F.Cu) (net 6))
 (segment (start 80.01 -308.61) (end 78.235 -308.61) (width 0.25) (layer B.Cu) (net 6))
 (via (at 80.01 -310.515) (size 0.8) (drill 0.4) (layers F.Cu B.Cu) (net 8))
 (segment (start 81.28 -311.785) (end 82.425 -311.785) (width 0.25) (layer F.Cu) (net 8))
 (segment (start 80.01 -310.515) (end 81.28 -311.785) (width 0.25) (layer F.Cu) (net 8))
 (segment (start 78.86 -313.055) (end 78.235 -313.055) (width 0.25) (layer B.Cu) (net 8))
 (segment (start 80.01 -311.905) (end 78.86 -313.055) (width 0.25) (layer B.Cu) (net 8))
 (segment (start 80.01 -310.515) (end 80.01 -311.905) (width 0.25) (layer B.Cu) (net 8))
 (segment (start 78.86 -313.065) (end 78.235 -313.69) (width 0.25) (layer B.Cu) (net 8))
 (segment (start 78.86 -313.055) (end 78.86 -313.065) (width 0.25) (layer B.Cu) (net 8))
 (segment (start 65.9 -312.055) (end 65.535 -312.42) (width 0.25) (layer B.Cu) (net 2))
 (segment (start 68.58 -312.055) (end 65.9 -312.055) (width 0.25) (layer B.Cu) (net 2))
 (segment (start 78.74 -312.65) (end 77.875 -311.785) (width 0.25) (layer F.Cu) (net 2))
 (segment (start 77.875 -311.785) (end 76.325 -311.785) (width 0.25) (layer F.Cu) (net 2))
 (segment (start 76.325 -311.785) (end 73.66 -311.785) (width 0.25) (layer F.Cu) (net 2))
 (segment (start 73.39 -312.055) (end 68.58 -312.055) (width 0.25) (layer F.Cu) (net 2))
 (segment (start 73.66 -311.785) (end 73.39 -312.055) (width 0.25) (layer F.Cu) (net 2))
 (segment (start 73.105 -316.31) (end 75.09 -314.325) (width 0.25) (layer F.Cu) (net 2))
 (segment (start 73.105 -316.45) (end 73.105 -316.31) (width 0.25) (layer F.Cu) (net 2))
 (segment (start 75.09 -314.325) (end 78.105 -314.325) (width 0.25) (layer F.Cu) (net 2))
 (segment (start 78.74 -313.69) (end 78.74 -312.65) (width 0.25) (layer F.Cu) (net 2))
 (segment (start 78.105 -314.325) (end 78.74 -313.69) (width 0.25) (layer F.Cu) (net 2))
 (segment (start 74.14 -313.055) (end 70.45104 -313.055) (width 0.25) (layer F.Cu) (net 1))
 (segment (start 69.18104 -313.055) (end 68.58 -313.055) (width 0.25) (layer F.Cu) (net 1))
 (segment (start 69.18104 -313.055) (end 70.485 -313.055) (width 0.25) (layer F.Cu) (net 1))
 (segment (start 66.04 -314.325) (end 65.535 -314.325) (width 0.25) (layer B.Cu) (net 1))
 (segment (start 67.44 -313.055) (end 65.535 -314.96) (width 0.25) (layer B.Cu) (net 1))
 (segment (start 68.58 -313.055) (end 67.44 -313.055) (width 0.25) (layer B.Cu) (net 1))
 (segment (start 74.14 -313.055) (end 76.325 -313.055) (width 0.25) (layer F.Cu) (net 1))
 (segment (start 74.775 -313.055) (end 76.325 -313.055) (width 0.25) (layer F.Cu) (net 1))
 (segment (start 72.505 -315.325) (end 74.775 -313.055) (width 0.25) (layer F.Cu) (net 1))
 (segment (start 72.505 -316.45) (end 72.505 -315.325) (width 0.25) (layer F.Cu) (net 1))
 (segment (start 64.43 -304.055) (end 64.43 -306.04) (width 0.25) (layer F.Cu) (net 10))
 (segment (start 64.43 -306.04) (end 64.43 -307.34) (width 0.25) (layer F.Cu) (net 10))
 (segment (start 63.905 -303.53) (end 64.43 -304.055) (width 0.25) (layer F.Cu) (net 10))
 (segment (start 63.23 -303.53) (end 63.905 -303.53) (width 0.25) (layer F.Cu) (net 10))
 (via (at 70.485 -314.96) (size 0.8) (drill 0.4) (layers F.Cu B.Cu) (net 13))
 (segment (start 71.305 -315.78) (end 70.485 -314.96) (width 0.25) (layer F.Cu) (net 13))
 (segment (start 71.305 -316.45) (end 71.305 -315.78) (width 0.25) (layer F.Cu) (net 13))
 (segment (start 69.18104 -308.055) (end 68.58 -308.055) (width 0.25) (layer B.Cu) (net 13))
 (segment (start 68.58 -308.055) (end 70.405 -308.055) (width 0.25) (layer B.Cu) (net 13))
 (segment (start 70.485 -313.69) (end 70.485 -314.96) (width 0.25) (layer B.Cu) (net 13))
 (segment (start 71.755 -312.42) (end 70.485 -313.69) (width 0.25) (layer B.Cu) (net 13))
 (segment (start 71.12 -308.105) (end 71.625 -308.61) (width 0.25) (layer B.Cu) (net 13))
 (segment (start 71.755 -308.61) (end 71.755 -312.42) (width 0.25) (layer B.Cu) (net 13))
 (segment (start 71.625 -308.61) (end 71.755 -308.61) (width 0.25) (layer B.Cu) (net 13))
 (segment (start 69.18104 -309.055) (end 68.58 -309.055) (width 0.25) (layer B.Cu) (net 12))
 (segment (start 69.81 -309.055) (end 69.18104 -309.055) (width 0.25) (layer B.Cu) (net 12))
 (segment (start 70.805 -310.05) (end 69.81 -309.055) (width 0.25) (layer B.Cu) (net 12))
 (segment (start 70.805 -310.5) (end 70.805 -310.05) (width 0.25) (layer B.Cu) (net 12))
 (segment (start 67.97896 -309.055) (end 66.26396 -307.34) (width 0.25) (layer B.Cu) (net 12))
 (segment (start 66.26396 -307.34) (end 65.535 -307.34) (width 0.25) (layer B.Cu) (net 12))
 (segment (start 68.58 -309.055) (end 67.97896 -309.055) (width 0.25) (layer B.Cu) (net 12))
 (segment (start 68.675 -311.15) (end 68.58 -311.055) (width 0.25) (layer F.Cu) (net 3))
 (segment (start 68.545 -311.02) (end 68.58 -311.055) (width 0.25) (layer F.Cu) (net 3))
 (segment (start 69.85 -311.055) (end 68.58 -311.055) (width 0.25) (layer F.Cu) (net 3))
 (segment (start 70.39 -310.515) (end 76.325 -310.515) (width 0.25) (layer F.Cu) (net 3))
 (segment (start 69.85 -311.055) (end 70.39 -310.515) (width 0.25) (layer F.Cu) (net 3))
 (segment (start 66.58 -311.055) (end 65.535 -310.01) (width 0.25) (layer B.Cu) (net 3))
 (segment (start 68.58 -311.055) (end 66.58 -311.055) (width 0.25) (layer B.Cu) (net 3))
 (segment (start 65.535 -310.01) (end 65.535 -309.88) (width 0.25) (layer B.Cu) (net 3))
 (via (at 73.025 -320.675) (size 0.8) (drill 0.4) (layers F.Cu B.Cu) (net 17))
 (segment (start 72.505 -320.155) (end 73.025 -320.675) (width 0.25) (layer F.Cu) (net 17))
 (segment (start 72.505 -318.55) (end 72.505 -320.155) (width 0.25) (layer F.Cu) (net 17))
 (segment (start 82.55 -319.525) (end 82.55 -318.9) (width 0.25) (layer B.Cu) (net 17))
 (segment (start 81.4 -320.675) (end 82.55 -319.525) (width 0.25) (layer B.Cu) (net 17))
 (segment (start 73.025 -320.675) (end 80.13 -320.675) (width 0.25) (layer B.Cu) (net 17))
 (segment (start 81.4 -320.675) (end 80.13 -320.675) (width 0.25) (layer B.Cu) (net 17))
 (segment (start 75.695 -318.9) (end 75.565 -318.77) (width 0.25) (layer B.Cu) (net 18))
 (segment (start 78.74 -318.9) (end 75.695 -318.9) (width 0.25) (layer B.Cu) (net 18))
 (segment (start 78.74 -318.9) (end 80.01 -318.9) (width 0.25) (layer B.Cu) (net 18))
 (via (at 74.295 -319.405) (size 0.8) (drill 0.4) (layers F.Cu B.Cu) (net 18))
 (segment (start 73.105 -318.55) (end 73.105 -318.69) (width 0.25) (layer F.Cu) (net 18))
 (segment (start 73.105 -318.69) (end 73.82 -319.405) (width 0.25) (layer F.Cu) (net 18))
 (segment (start 73.82 -319.405) (end 74.295 -319.405) (width 0.25) (layer F.Cu) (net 18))
 (segment (start 74.8 -318.9) (end 74.295 -319.405) (width 0.25) (layer B.Cu) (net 18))
 (segment (start 76.2 -318.9) (end 74.8 -318.9) (width 0.25) (layer B.Cu) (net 18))
 (segment (start 70.705 -318.55) (end 71.305 -318.55) (width 0.25) (layer F.Cu) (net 15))
 (segment (start 70.705 -318.55) (end 70.705 -319.445) (width 0.25) (layer F.Cu) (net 15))
 (segment (start 69.345 -320.805) (end 66.04 -320.805) (width 0.25) (layer F.Cu) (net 15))
 (segment (start 70.705 -319.445) (end 69.345 -320.805) (width 0.25) (layer F.Cu) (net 15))
 (segment (start 66.04 -320.805) (end 62.865 -320.805) (width 0.25) (layer F.Cu) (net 15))
 (via (at 71.12 -320.675) (size 0.8) (drill 0.4) (layers F.Cu B.Cu) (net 16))
 (segment (start 71.905 -319.89) (end 71.12 -320.675) (width 0.25) (layer F.Cu) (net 16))
 (segment (start 71.905 -318.55) (end 71.905 -319.89) (width 0.25) (layer F.Cu) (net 16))
 (segment (start 71.12 -320.675) (end 71.905 -319.89) (width 0.25) (layer B.Cu) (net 16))
 (segment (start 73.025 -318.77) (end 71.12 -320.675) (width 0.25) (layer B.Cu) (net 16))
 (segment (start 73.66 -311.644998) (end 73.66 -318.135) (width 0.25) (layer B.Cu) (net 16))
 (segment (start 73.66 -318.135) (end 73.025 -318.77) (width 0.25) (layer B.Cu) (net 16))
 (segment (start 72.705 -311.15) (end 73.165002 -311.15) (width 0.25) (layer B.Cu) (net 16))
 (segment (start 73.165002 -311.15) (end 73.66 -311.644998) (width 0.25) (layer B.Cu) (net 16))
 (segment (start 60.96 -313.055) (end 60.96 -310.515) (width 0.25) (layer F.Cu) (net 11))
 (segment (start 60.03 -309.705) (end 60.84 -310.515) (width 0.25) (layer F.Cu) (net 11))
 (segment (start 60.03 -307.34) (end 60.03 -309.705) (width 0.25) (layer F.Cu) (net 11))
 (segment (start 60.03 -304.46) (end 60.03 -307.34) (width 0.25) (layer F.Cu) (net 11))
 (segment (start 68.58 -304.8) (end 66.04 -302.26) (width 0.25) (layer F.Cu) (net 11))
 (segment (start 66.04 -302.26) (end 60.96 -302.26) (width 0.25) (layer F.Cu) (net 11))
 (segment (start 68.58 -307.055) (end 68.58 -304.8) (width 0.25) (layer F.Cu) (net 11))
 (segment (start 60.96 -302.26) (end 60.03 -303.19) (width 0.25) (layer F.Cu) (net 11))
 (segment (start 60.03 -303.19) (end 60.03 -304.46) (width 0.25) (layer F.Cu) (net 11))
 (segment (start 71.755 -314.325) (end 71.905 -314.461263) (width 0.25) (layer F.Cu) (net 14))
 (via (at 71.755 -314.325) (size 0.8) (drill 0.4) (layers F.Cu B.Cu) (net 14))
 (segment (start 71.905 -314.461263) (end 71.905 -316.45) (width 0.25) (layer F.Cu) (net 14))
 (segment (start 71.755 -314.325) (end 71.755 -317.235) (width 0.25) (layer B.Cu) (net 14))
 (segment (start 70.22 -318.77) (end 68.58 -318.77) (width 0.25) (layer B.Cu) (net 14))
 (segment (start 71.755 -317.235) (end 70.22 -318.77) (width 0.25) (layer B.Cu) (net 14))
 (segment (start 68.58 -318.77) (end 66.04 -318.77) (width 0.25) (layer B.Cu) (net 14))
 (via (at 66.04 -318.77) (size 0.8) (drill 0.4) (layers F.Cu B.Cu) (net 14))
 (segment (start 65.275 -318.005) (end 66.04 -318.77) (width 0.25) (layer F.Cu) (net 14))
 (segment (start 62.865 -318.005) (end 65.275 -318.005) (width 0.25) (layer F.Cu) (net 14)))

